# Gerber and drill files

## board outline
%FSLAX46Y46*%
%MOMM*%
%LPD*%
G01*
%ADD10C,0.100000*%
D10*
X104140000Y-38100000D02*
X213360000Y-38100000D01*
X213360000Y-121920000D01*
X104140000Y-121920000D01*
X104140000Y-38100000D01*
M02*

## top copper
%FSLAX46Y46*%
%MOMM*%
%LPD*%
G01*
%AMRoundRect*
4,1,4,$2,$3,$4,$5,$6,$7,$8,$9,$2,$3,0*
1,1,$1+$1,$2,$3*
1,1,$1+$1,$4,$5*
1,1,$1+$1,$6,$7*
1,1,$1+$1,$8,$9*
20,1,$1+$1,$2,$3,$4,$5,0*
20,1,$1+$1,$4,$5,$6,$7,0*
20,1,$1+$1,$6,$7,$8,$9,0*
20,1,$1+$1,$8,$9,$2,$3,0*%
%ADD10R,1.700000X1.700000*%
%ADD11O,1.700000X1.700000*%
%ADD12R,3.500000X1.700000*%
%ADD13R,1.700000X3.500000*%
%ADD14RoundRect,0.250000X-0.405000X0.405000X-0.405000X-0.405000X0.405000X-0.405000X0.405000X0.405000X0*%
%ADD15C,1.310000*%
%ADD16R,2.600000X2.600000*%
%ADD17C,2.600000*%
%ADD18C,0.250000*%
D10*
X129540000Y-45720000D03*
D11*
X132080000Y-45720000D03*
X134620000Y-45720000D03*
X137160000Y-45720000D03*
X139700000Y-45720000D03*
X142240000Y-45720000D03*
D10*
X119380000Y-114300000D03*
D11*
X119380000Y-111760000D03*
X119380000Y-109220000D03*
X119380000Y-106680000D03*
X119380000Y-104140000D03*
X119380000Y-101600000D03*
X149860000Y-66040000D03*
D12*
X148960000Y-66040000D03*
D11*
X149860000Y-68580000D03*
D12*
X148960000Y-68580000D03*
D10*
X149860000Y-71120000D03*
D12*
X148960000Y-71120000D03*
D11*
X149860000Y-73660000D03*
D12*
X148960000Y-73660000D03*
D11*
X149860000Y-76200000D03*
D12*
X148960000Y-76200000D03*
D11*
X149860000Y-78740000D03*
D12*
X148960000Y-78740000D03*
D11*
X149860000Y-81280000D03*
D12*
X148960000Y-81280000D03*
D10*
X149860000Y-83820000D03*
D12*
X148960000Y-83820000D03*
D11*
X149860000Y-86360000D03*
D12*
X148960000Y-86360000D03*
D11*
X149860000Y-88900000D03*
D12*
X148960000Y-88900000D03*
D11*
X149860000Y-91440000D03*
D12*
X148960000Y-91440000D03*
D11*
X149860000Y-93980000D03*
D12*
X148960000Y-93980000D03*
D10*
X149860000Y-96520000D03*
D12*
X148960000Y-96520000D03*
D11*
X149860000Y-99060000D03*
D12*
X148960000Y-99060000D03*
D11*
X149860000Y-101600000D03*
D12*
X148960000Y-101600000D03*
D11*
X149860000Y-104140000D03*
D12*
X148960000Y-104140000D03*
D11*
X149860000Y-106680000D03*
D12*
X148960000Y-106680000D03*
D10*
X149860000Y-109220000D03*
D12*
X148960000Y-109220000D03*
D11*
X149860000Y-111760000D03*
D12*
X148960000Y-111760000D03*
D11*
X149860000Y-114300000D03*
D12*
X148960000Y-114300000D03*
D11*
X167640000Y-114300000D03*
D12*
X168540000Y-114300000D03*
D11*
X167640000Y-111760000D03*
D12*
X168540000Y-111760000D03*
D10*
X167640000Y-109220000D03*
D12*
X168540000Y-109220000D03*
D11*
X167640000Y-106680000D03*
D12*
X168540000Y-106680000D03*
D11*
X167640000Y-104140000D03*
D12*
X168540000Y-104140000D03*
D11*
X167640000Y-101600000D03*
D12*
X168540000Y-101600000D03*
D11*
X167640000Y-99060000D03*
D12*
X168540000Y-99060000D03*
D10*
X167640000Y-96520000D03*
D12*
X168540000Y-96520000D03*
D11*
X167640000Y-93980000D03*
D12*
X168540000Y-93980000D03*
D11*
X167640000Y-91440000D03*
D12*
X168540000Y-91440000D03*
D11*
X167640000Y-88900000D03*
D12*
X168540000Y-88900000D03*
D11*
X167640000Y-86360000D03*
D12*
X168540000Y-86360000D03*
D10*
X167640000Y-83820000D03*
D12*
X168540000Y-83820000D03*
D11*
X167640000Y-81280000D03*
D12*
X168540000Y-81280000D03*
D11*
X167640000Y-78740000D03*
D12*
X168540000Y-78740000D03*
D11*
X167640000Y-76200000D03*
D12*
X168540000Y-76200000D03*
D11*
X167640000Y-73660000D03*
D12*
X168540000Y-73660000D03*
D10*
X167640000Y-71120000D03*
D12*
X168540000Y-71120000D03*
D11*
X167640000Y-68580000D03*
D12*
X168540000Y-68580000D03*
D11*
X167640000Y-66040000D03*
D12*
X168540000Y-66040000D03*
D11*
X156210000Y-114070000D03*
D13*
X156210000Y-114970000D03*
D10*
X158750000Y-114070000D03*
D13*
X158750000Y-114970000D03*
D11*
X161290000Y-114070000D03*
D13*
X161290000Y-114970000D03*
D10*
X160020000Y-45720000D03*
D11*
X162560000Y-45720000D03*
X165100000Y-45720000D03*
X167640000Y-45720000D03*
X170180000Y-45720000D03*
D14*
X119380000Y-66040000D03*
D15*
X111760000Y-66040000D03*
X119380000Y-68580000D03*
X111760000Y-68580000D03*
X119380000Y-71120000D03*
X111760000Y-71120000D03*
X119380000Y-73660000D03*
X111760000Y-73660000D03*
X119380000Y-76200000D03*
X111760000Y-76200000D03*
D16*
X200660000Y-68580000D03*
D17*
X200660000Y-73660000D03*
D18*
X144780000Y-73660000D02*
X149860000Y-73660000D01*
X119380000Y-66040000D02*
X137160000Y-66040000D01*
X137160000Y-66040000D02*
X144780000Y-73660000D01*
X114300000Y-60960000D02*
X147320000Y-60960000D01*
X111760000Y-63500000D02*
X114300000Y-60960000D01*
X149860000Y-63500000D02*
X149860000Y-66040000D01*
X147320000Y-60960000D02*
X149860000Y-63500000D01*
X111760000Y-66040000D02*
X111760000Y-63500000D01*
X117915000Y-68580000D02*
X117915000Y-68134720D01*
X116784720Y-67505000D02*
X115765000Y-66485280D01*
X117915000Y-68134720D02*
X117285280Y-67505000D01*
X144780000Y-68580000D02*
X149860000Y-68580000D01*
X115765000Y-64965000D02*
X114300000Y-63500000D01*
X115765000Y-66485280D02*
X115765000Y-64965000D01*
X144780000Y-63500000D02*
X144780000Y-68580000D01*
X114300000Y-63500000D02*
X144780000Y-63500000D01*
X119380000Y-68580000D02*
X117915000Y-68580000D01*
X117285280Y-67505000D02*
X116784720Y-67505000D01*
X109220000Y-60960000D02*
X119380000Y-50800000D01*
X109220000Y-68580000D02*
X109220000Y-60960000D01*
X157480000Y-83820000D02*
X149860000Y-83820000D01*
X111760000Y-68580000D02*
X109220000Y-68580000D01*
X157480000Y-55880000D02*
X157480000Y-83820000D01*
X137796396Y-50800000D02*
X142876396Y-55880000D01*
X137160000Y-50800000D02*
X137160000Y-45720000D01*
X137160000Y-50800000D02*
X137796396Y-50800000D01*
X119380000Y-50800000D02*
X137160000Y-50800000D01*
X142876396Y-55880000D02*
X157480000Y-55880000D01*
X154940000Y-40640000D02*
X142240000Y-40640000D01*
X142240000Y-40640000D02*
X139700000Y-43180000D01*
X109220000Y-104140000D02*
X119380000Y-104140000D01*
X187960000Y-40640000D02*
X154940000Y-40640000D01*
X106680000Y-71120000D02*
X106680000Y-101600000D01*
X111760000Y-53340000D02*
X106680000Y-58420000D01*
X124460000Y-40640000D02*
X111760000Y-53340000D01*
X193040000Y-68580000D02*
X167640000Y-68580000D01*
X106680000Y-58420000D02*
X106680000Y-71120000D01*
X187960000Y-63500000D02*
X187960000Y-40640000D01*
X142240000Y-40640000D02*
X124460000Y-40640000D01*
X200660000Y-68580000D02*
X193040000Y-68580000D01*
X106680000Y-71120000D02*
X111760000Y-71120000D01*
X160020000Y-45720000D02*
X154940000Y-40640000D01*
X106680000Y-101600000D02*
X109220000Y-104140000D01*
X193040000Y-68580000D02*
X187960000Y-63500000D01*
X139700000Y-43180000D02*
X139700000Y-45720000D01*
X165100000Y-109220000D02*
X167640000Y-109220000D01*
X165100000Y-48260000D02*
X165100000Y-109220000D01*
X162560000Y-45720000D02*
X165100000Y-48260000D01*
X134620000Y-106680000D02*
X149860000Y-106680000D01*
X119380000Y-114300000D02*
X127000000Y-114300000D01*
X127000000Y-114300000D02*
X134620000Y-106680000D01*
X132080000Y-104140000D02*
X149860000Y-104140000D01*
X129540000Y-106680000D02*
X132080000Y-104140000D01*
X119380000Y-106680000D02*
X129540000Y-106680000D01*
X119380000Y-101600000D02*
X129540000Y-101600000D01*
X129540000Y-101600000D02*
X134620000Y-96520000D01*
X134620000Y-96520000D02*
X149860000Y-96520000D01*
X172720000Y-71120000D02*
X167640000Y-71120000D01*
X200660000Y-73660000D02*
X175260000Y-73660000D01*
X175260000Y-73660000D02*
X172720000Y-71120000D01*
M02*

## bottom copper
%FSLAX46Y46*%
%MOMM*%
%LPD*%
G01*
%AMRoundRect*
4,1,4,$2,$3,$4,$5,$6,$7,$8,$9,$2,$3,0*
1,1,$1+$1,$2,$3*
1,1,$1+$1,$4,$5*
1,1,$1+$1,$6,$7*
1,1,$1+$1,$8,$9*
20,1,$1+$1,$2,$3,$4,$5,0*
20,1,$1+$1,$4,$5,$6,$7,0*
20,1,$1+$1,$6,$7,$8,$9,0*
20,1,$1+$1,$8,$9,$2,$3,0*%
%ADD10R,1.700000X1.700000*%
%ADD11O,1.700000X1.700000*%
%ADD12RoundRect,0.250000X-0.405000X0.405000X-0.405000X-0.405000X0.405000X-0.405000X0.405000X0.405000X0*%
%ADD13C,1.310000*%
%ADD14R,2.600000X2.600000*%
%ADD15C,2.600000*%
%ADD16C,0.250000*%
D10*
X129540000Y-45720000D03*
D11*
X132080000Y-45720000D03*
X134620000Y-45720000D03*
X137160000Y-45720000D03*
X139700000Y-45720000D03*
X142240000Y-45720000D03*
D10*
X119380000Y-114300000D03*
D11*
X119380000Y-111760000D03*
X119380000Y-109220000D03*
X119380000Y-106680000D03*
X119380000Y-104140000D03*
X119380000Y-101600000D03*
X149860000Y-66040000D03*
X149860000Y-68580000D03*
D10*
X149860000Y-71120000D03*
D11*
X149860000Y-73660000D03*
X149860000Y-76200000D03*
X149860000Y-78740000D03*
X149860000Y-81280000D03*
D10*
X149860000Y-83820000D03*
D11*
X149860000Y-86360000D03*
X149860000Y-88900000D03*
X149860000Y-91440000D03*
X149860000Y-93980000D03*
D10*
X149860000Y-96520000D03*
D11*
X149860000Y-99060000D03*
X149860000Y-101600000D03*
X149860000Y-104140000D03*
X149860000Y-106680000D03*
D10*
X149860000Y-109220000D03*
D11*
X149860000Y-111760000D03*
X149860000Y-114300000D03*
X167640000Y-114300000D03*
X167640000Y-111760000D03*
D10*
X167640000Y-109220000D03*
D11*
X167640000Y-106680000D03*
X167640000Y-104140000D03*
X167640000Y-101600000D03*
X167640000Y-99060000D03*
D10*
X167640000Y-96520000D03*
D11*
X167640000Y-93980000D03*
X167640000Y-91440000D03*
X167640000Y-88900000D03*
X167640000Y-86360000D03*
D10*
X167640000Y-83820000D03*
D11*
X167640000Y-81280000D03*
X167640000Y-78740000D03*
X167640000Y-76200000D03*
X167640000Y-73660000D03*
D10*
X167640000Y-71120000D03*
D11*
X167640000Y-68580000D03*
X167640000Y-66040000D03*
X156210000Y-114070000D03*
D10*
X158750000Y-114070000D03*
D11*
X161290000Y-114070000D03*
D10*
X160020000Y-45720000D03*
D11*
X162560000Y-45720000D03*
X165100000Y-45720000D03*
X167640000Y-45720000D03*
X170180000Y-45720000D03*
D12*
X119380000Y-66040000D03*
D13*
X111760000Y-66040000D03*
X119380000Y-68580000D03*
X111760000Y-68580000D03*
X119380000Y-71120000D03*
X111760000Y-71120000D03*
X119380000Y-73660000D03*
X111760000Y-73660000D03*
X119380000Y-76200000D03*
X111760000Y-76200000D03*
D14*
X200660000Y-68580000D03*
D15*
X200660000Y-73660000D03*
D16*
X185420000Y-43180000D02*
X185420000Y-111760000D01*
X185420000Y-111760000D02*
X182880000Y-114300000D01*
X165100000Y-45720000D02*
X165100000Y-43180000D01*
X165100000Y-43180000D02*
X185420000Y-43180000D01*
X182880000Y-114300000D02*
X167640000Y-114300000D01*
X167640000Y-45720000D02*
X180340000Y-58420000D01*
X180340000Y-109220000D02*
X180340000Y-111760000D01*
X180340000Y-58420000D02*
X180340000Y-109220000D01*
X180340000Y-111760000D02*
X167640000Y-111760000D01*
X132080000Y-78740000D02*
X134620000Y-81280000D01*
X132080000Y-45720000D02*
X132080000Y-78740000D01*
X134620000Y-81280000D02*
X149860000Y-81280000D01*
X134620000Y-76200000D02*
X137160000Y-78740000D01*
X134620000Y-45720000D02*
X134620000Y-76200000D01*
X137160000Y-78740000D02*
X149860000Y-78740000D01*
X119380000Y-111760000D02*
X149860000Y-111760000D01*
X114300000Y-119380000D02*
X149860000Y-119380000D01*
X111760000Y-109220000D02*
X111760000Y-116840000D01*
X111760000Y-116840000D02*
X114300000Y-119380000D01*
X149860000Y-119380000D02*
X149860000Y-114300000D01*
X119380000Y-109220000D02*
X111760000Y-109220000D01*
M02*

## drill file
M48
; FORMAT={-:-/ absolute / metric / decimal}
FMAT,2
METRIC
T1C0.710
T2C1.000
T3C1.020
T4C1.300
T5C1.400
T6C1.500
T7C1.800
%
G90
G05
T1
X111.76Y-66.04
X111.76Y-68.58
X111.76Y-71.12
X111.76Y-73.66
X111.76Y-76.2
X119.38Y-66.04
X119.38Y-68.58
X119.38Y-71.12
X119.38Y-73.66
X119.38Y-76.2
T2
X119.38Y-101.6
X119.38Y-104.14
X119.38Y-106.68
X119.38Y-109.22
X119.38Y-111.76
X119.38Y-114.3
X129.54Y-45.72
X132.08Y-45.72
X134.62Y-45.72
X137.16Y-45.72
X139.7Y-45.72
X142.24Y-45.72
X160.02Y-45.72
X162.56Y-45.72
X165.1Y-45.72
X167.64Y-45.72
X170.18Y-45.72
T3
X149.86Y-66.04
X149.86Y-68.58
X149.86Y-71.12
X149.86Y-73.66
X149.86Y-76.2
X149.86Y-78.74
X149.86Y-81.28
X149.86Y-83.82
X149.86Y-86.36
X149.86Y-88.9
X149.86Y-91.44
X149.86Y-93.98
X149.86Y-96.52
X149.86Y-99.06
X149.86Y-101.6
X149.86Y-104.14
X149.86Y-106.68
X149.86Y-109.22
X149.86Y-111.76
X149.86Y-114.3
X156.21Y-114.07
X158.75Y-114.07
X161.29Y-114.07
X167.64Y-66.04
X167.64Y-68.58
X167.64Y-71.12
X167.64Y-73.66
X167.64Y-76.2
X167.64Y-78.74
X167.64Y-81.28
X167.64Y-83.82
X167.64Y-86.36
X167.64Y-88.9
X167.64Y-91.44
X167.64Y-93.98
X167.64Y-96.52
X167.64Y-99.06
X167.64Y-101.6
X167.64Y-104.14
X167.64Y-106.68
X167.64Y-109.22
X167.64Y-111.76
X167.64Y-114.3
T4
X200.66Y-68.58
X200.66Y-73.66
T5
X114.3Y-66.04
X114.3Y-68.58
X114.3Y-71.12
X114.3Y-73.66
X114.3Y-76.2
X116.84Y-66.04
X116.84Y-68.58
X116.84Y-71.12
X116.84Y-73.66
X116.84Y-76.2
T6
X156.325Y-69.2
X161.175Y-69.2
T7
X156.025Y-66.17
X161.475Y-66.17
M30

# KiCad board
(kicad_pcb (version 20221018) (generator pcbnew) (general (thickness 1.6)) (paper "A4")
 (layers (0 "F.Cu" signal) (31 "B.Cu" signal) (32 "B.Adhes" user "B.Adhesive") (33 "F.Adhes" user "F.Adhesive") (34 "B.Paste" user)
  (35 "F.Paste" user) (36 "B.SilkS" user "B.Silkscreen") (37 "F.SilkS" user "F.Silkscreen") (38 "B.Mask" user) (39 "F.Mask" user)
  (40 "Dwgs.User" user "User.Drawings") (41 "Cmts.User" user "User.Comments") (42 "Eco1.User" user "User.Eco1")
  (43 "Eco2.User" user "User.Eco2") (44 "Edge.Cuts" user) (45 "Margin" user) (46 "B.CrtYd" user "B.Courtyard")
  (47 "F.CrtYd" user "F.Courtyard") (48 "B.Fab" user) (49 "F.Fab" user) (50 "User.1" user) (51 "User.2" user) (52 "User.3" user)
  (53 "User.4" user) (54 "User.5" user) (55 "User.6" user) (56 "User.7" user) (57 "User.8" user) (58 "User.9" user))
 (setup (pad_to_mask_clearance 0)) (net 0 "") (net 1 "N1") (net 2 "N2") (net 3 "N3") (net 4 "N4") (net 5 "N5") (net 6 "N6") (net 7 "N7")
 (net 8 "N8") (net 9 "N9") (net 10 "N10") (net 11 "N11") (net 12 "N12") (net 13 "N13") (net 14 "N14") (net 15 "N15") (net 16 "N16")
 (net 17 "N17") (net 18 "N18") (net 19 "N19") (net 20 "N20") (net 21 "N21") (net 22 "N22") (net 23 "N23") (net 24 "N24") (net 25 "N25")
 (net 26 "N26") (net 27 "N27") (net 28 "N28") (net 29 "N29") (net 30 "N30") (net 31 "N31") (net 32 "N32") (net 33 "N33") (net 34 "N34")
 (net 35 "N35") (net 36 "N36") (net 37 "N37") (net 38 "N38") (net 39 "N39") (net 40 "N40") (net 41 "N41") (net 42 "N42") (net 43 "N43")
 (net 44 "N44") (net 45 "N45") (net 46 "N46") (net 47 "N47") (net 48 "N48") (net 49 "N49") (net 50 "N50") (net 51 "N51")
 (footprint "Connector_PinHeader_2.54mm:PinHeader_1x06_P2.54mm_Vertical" (layer "F.Cu") (at 129.54 45.72 90)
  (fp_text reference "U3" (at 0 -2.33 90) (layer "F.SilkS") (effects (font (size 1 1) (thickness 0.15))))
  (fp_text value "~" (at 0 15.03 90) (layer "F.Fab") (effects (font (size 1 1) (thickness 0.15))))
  (pad "1" thru_hole rect (at 0 0 90) (size 1.7 1.7) (drill 1) (layers "*.Cu" "*.Mask") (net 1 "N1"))
  (pad "2" thru_hole oval (at 0 2.54 90) (size 1.7 1.7) (drill 1) (layers "*.Cu" "*.Mask") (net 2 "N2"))
  (pad "3" thru_hole oval (at 0 5.08 90) (size 1.7 1.7) (drill 1) (layers "*.Cu" "*.Mask") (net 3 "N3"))
  (pad "4" thru_hole oval (at 0 7.62 90) (size 1.7 1.7) (drill 1) (layers "*.Cu" "*.Mask") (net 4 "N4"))
  (pad "5" thru_hole oval (at 0 10.16 90) (size 1.7 1.7) (drill 1) (layers "*.Cu" "*.Mask") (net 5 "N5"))
  (pad "6" thru_hole oval (at 0 12.7 90) (size 1.7 1.7) (drill 1) (layers "*.Cu" "*.Mask") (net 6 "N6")))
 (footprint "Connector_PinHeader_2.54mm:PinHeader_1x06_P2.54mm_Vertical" (layer "F.Cu") (at 119.38 114.3 180)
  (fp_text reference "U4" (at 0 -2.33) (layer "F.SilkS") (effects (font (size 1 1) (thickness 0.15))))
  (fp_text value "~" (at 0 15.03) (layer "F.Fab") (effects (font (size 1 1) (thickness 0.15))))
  (pad "1" thru_hole rect (at 0 0 180) (size 1.7 1.7) (drill 1) (layers "*.Cu" "*.Mask") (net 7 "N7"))
  (pad "2" thru_hole oval (at 0 2.54 180) (size 1.7 1.7) (drill 1) (layers "*.Cu" "*.Mask") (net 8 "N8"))
  (pad "3" thru_hole oval (at 0 5.08 180) (size 1.7 1.7) (drill 1) (layers "*.Cu" "*.Mask") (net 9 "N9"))
  (pad "4" thru_hole oval (at 0 7.62 180) (size 1.7 1.7) (drill 1) (layers "*.Cu" "*.Mask") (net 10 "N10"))
  (pad "5" thru_hole oval (at 0 10.16 180) (size 1.7 1.7) (drill 1) (layers "*.Cu" "*.Mask") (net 5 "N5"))
  (pad "6" thru_hole oval (at 0 12.7 180) (size 1.7 1.7) (drill 1) (layers "*.Cu" "*.Mask") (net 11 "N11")))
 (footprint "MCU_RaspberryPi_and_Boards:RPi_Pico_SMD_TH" (layer "F.Cu") (at 158.75 90.17)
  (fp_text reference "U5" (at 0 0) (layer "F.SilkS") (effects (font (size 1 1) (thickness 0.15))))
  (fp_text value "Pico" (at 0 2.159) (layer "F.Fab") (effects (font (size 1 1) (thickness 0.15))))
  (pad "" np_thru_hole oval (at -2.725 -24) (size 1.8 1.8) (drill 1.8) (layers "*.Cu" "*.Mask"))
  (pad "" np_thru_hole oval (at -2.425 -20.97) (size 1.5 1.5) (drill 1.5) (layers "*.Cu" "*.Mask"))
  (pad "" np_thru_hole oval (at 2.425 -20.97) (size 1.5 1.5) (drill 1.5) (layers "*.Cu" "*.Mask"))
  (pad "" np_thru_hole oval (at 2.725 -24) (size 1.8 1.8) (drill 1.8) (layers "*.Cu" "*.Mask"))
  (pad "1" thru_hole oval (at -8.89 -24.13) (size 1.7 1.7) (drill 1.02) (layers "*.Cu" "*.Mask") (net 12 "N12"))
  (pad "1" smd rect (at -8.89 -24.13) (size 3.5 1.7) (drill (offset -0.9 0)) (layers "F.Cu" "F.Mask") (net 12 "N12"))
  (pad "2" thru_hole oval (at -8.89 -21.59) (size 1.7 1.7) (drill 1.02) (layers "*.Cu" "*.Mask") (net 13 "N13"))
  (pad "2" smd rect (at -8.89 -21.59) (size 3.5 1.7) (drill (offset -0.9 0)) (layers "F.Cu" "F.Mask") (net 13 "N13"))
  (pad "3" thru_hole rect (at -8.89 -19.05) (size 1.7 1.7) (drill 1.02) (layers "*.Cu" "*.Mask") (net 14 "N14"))
  (pad "3" smd rect (at -8.89 -19.05) (size 3.5 1.7) (drill (offset -0.9 0)) (layers "F.Cu" "F.Mask") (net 14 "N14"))
  (pad "4" thru_hole oval (at -8.89 -16.51) (size 1.7 1.7) (drill 1.02) (layers "*.Cu" "*.Mask") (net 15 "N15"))
  (pad "4" smd rect (at -8.89 -16.51) (size 3.5 1.7) (drill (offset -0.9 0)) (layers "F.Cu" "F.Mask") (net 15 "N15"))
  (pad "5" thru_hole oval (at -8.89 -13.97) (size 1.7 1.7) (drill 1.02) (layers "*.Cu" "*.Mask") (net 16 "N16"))
  (pad "5" smd rect (at -8.89 -13.97) (size 3.5 1.7) (drill (offset -0.9 0)) (layers "F.Cu" "F.Mask") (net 16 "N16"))
  (pad "6" thru_hole oval (at -8.89 -11.43) (size 1.7 1.7) (drill 1.02) (layers "*.Cu" "*.Mask") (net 3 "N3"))
  (pad "6" smd rect (at -8.89 -11.43) (size 3.5 1.7) (drill (offset -0.9 0)) (layers "F.Cu" "F.Mask") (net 3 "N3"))
  (pad "7" thru_hole oval (at -8.89 -8.89) (size 1.7 1.7) (drill 1.02) (layers "*.Cu" "*.Mask") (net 2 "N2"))
  (pad "7" smd rect (at -8.89 -8.89) (size 3.5 1.7) (drill (offset -0.9 0)) (layers "F.Cu" "F.Mask") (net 2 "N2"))
  (pad "8" thru_hole rect (at -8.89 -6.35) (size 1.7 1.7) (drill 1.02) (layers "*.Cu" "*.Mask") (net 4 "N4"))
  (pad "8" smd rect (at -8.89 -6.35) (size 3.5 1.7) (drill (offset -0.9 0)) (layers "F.Cu" "F.Mask") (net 4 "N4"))
  (pad "9" thru_hole oval (at -8.89 -3.81) (size 1.7 1.7) (drill 1.02) (layers "*.Cu" "*.Mask") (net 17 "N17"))
  (pad "9" smd rect (at -8.89 -3.81) (size 3.5 1.7) (drill (offset -0.9 0)) (layers "F.Cu" "F.Mask") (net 17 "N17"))
  (pad "10" thru_hole oval (at -8.89 -1.27) (size 1.7 1.7) (drill 1.02) (layers "*.Cu" "*.Mask") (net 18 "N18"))
  (pad "10" smd rect (at -8.89 -1.27) (size 3.5 1.7) (drill (offset -0.9 0)) (layers "F.Cu" "F.Mask") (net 18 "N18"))
  (pad "11" thru_hole oval (at -8.89 1.27) (size 1.7 1.7) (drill 1.02) (layers "*.Cu" "*.Mask") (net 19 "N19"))
  (pad "11" smd rect (at -8.89 1.27) (size 3.5 1.7) (drill (offset -0.9 0)) (layers "F.Cu" "F.Mask") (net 19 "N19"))
  (pad "12" thru_hole oval (at -8.89 3.81) (size 1.7 1.7) (drill 1.02) (layers "*.Cu" "*.Mask") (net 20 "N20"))
  (pad "12" smd rect (at -8.89 3.81) (size 3.5 1.7) (drill (offset -0.9 0)) (layers "F.Cu" "F.Mask") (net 20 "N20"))
  (pad "13" thru_hole rect (at -8.89 6.35) (size 1.7 1.7) (drill 1.02) (layers "*.Cu" "*.Mask") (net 11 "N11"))
  (pad "13" smd rect (at -8.89 6.35) (size 3.5 1.7) (drill (offset -0.9 0)) (layers "F.Cu" "F.Mask") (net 11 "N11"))
  (pad "14" thru_hole oval (at -8.89 8.89) (size 1.7 1.7) (drill 1.02) (layers "*.Cu" "*.Mask") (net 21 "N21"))
  (pad "14" smd rect (at -8.89 8.89) (size 3.5 1.7) (drill (offset -0.9 0)) (layers "F.Cu" "F.Mask") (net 21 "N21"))
  (pad "15" thru_hole oval (at -8.89 11.43) (size 1.7 1.7) (drill 1.02) (layers "*.Cu" "*.Mask") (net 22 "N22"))
  (pad "15" smd rect (at -8.89 11.43) (size 3.5 1.7) (drill (offset -0.9 0)) (layers "F.Cu" "F.Mask") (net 22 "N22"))
  (pad "16" thru_hole oval (at -8.89 13.97) (size 1.7 1.7) (drill 1.02) (layers "*.Cu" "*.Mask") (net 10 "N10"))
  (pad "16" smd rect (at -8.89 13.97) (size 3.5 1.7) (drill (offset -0.9 0)) (layers "F.Cu" "F.Mask") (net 10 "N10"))
  (pad "17" thru_hole oval (at -8.89 16.51) (size 1.7 1.7) (drill 1.02) (layers "*.Cu" "*.Mask") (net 7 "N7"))
  (pad "17" smd rect (at -8.89 16.51) (size 3.5 1.7) (drill (offset -0.9 0)) (layers "F.Cu" "F.Mask") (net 7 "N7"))
  (pad "18" thru_hole rect (at -8.89 19.05) (size 1.7 1.7) (drill 1.02) (layers "*.Cu" "*.Mask") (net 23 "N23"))
  (pad "18" smd rect (at -8.89 19.05) (size 3.5 1.7) (drill (offset -0.9 0)) (layers "F.Cu" "F.Mask") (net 23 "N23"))
  (pad "19" thru_hole oval (at -8.89 21.59) (size 1.7 1.7) (drill 1.02) (layers "*.Cu" "*.Mask") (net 8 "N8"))
  (pad "19" smd rect (at -8.89 21.59) (size 3.5 1.7) (drill (offset -0.9 0)) (layers "F.Cu" "F.Mask") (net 8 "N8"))
  (pad "20" thru_hole oval (at -8.89 24.13) (size 1.7 1.7) (drill 1.02) (layers "*.Cu" "*.Mask") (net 9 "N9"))
  (pad "20" smd rect (at -8.89 24.13) (size 3.5 1.7) (drill (offset -0.9 0)) (layers "F.Cu" "F.Mask") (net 9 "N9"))
  (pad "21" thru_hole oval (at 8.89 24.13) (size 1.7 1.7) (drill 1.02) (layers "*.Cu" "*.Mask") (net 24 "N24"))
  (pad "21" smd rect (at 8.89 24.13) (size 3.5 1.7) (drill (offset 0.9 0)) (layers "F.Cu" "F.Mask") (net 24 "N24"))
  (pad "22" thru_hole oval (at 8.89 21.59) (size 1.7 1.7) (drill 1.02) (layers "*.Cu" "*.Mask") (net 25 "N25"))
  (pad "22" smd rect (at 8.89 21.59) (size 3.5 1.7) (drill (offset 0.9 0)) (layers "F.Cu" "F.Mask") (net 25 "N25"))
  (pad "23" thru_hole rect (at 8.89 19.05) (size 1.7 1.7) (drill 1.02) (layers "*.Cu" "*.Mask") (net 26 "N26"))
  (pad "23" smd rect (at 8.89 19.05) (size 3.5 1.7) (drill (offset 0.9 0)) (layers "F.Cu" "F.Mask") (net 26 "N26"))
  (pad "24" thru_hole oval (at 8.89 16.51) (size 1.7 1.7) (drill 1.02) (layers "*.Cu" "*.Mask") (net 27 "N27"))
  (pad "24" smd rect (at 8.89 16.51) (size 3.5 1.7) (drill (offset 0.9 0)) (layers "F.Cu" "F.Mask") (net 27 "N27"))
  (pad "25" thru_hole oval (at 8.89 13.97) (size 1.7 1.7) (drill 1.02) (layers "*.Cu" "*.Mask") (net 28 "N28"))
  (pad "25" smd rect (at 8.89 13.97) (size 3.5 1.7) (drill (offset 0.9 0)) (layers "F.Cu" "F.Mask") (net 28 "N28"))
  (pad "26" thru_hole oval (at 8.89 11.43) (size 1.7 1.7) (drill 1.02) (layers "*.Cu" "*.Mask") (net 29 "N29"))
  (pad "26" smd rect (at 8.89 11.43) (size 3.5 1.7) (drill (offset 0.9 0)) (layers "F.Cu" "F.Mask") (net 29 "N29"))
  (pad "27" thru_hole oval (at 8.89 8.89) (size 1.7 1.7) (drill 1.02) (layers "*.Cu" "*.Mask") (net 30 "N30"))
  (pad "27" smd rect (at 8.89 8.89) (size 3.5 1.7) (drill (offset 0.9 0)) (layers "F.Cu" "F.Mask") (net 30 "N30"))
  (pad "28" thru_hole rect (at 8.89 6.35) (size 1.7 1.7) (drill 1.02) (layers "*.Cu" "*.Mask") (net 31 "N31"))
  (pad "28" smd rect (at 8.89 6.35) (size 3.5 1.7) (drill (offset 0.9 0)) (layers "F.Cu" "F.Mask") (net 31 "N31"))
  (pad "29" thru_hole oval (at 8.89 3.81) (size 1.7 1.7) (drill 1.02) (layers "*.Cu" "*.Mask") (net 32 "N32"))
  (pad "29" smd rect (at 8.89 3.81) (size 3.5 1.7) (drill (offset 0.9 0)) (layers "F.Cu" "F.Mask") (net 32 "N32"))
  (pad "30" thru_hole oval (at 8.89 1.27) (size 1.7 1.7) (drill 1.02) (layers "*.Cu" "*.Mask") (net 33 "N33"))
  (pad "30" smd rect (at 8.89 1.27) (size 3.5 1.7) (drill (offset 0.9 0)) (layers "F.Cu" "F.Mask") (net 33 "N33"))
  (pad "31" thru_hole oval (at 8.89 -1.27) (size 1.7 1.7) (drill 1.02) (layers "*.Cu" "*.Mask") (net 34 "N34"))
  (pad "31" smd rect (at 8.89 -1.27) (size 3.5 1.7) (drill (offset 0.9 0)) (layers "F.Cu" "F.Mask") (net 34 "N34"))
  (pad "32" thru_hole oval (at 8.89 -3.81) (size 1.7 1.7) (drill 1.02) (layers "*.Cu" "*.Mask") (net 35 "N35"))
  (pad "32" smd rect (at 8.89 -3.81) (size 3.5 1.7) (drill (offset 0.9 0)) (layers "F.Cu" "F.Mask") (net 35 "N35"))
  (pad "33" thru_hole rect (at 8.89 -6.35) (size 1.7 1.7) (drill 1.02) (layers "*.Cu" "*.Mask") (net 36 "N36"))
  (pad "33" smd rect (at 8.89 -6.35) (size 3.5 1.7) (drill (offset 0.9 0)) (layers "F.Cu" "F.Mask") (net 36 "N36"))
  (pad "34" thru_hole oval (at 8.89 -8.89) (size 1.7 1.7) (drill 1.02) (layers "*.Cu" "*.Mask") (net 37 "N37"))
  (pad "34" smd rect (at 8.89 -8.89) (size 3.5 1.7) (drill (offset 0.9 0)) (layers "F.Cu" "F.Mask") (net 37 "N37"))
  (pad "35" thru_hole oval (at 8.89 -11.43) (size 1.7 1.7) (drill 1.02) (layers "*.Cu" "*.Mask") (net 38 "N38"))
  (pad "35" smd rect (at 8.89 -11.43) (size 3.5 1.7) (drill (offset 0.9 0)) (layers "F.Cu" "F.Mask") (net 38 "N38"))
  (pad "36" thru_hole oval (at 8.89 -13.97) (size 1.7 1.7) (drill 1.02) (layers "*.Cu" "*.Mask") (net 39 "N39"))
  (pad "36" smd rect (at 8.89 -13.97) (size 3.5 1.7) (drill (offset 0.9 0)) (layers "F.Cu" "F.Mask") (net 39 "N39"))
  (pad "37" thru_hole oval (at 8.89 -16.51) (size 1.7 1.7) (drill 1.02) (layers "*.Cu" "*.Mask") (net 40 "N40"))
  (pad "37" smd rect (at 8.89 -16.51) (size 3.5 1.7) (drill (offset 0.9 0)) (layers "F.Cu" "F.Mask") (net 40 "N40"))
  (pad "38" thru_hole rect (at 8.89 -19.05) (size 1.7 1.7) (drill 1.02) (layers "*.Cu" "*.Mask") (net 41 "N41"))
  (pad "38" smd rect (at 8.89 -19.05) (size 3.5 1.7) (drill (offset 0.9 0)) (layers "F.Cu" "F.Mask") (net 41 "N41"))
  (pad "39" thru_hole oval (at 8.89 -21.59) (size 1.7 1.7) (drill 1.02) (layers "*.Cu" "*.Mask") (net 5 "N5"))
  (pad "39" smd rect (at 8.89 -21.59) (size 3.5 1.7) (drill (offset 0.9 0)) (layers "F.Cu" "F.Mask") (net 5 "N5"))
  (pad "40" thru_hole oval (at 8.89 -24.13) (size 1.7 1.7) (drill 1.02) (layers "*.Cu" "*.Mask") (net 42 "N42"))
  (pad "40" smd rect (at 8.89 -24.13) (size 3.5 1.7) (drill (offset 0.9 0)) (layers "F.Cu" "F.Mask") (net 42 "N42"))
  (pad "41" thru_hole oval (at -2.54 23.9) (size 1.7 1.7) (drill 1.02) (layers "*.Cu" "*.Mask") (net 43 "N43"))
  (pad "41" smd rect (at -2.54 23.9 90) (size 3.5 1.7) (drill (offset -0.9 0)) (layers "F.Cu" "F.Mask") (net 43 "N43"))
  (pad "42" thru_hole rect (at 0 23.9) (size 1.7 1.7) (drill 1.02) (layers "*.Cu" "*.Mask") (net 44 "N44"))
  (pad "42" smd rect (at 0 23.9 90) (size 3.5 1.7) (drill (offset -0.9 0)) (layers "F.Cu" "F.Mask") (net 44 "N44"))
  (pad "43" thru_hole oval (at 2.54 23.9) (size 1.7 1.7) (drill 1.02) (layers "*.Cu" "*.Mask") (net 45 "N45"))
  (pad "43" smd rect (at 2.54 23.9 90) (size 3.5 1.7) (drill (offset -0.9 0)) (layers "F.Cu" "F.Mask") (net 45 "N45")))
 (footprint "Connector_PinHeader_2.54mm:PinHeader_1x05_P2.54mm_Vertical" (layer "F.Cu") (at 160.02 45.72 90)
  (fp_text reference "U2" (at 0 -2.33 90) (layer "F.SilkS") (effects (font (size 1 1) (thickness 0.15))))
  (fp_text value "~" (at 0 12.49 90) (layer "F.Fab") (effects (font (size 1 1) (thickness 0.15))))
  (pad "1" thru_hole rect (at 0 0 90) (size 1.7 1.7) (drill 1) (layers "*.Cu" "*.Mask") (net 5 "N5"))
  (pad "2" thru_hole oval (at 0 2.54 90) (size 1.7 1.7) (drill 1) (layers "*.Cu" "*.Mask") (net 26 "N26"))
  (pad "3" thru_hole oval (at 0 5.08 90) (size 1.7 1.7) (drill 1) (layers "*.Cu" "*.Mask") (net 24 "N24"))
  (pad "4" thru_hole oval (at 0 7.62 90) (size 1.7 1.7) (drill 1) (layers "*.Cu" "*.Mask") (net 25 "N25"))
  (pad "5" thru_hole oval (at 0 10.16 90) (size 1.7 1.7) (drill 1) (layers "*.Cu" "*.Mask") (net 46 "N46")))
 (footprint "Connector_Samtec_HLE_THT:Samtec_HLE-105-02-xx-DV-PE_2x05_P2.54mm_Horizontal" (layer "F.Cu") (at 119.38 66.04 -90)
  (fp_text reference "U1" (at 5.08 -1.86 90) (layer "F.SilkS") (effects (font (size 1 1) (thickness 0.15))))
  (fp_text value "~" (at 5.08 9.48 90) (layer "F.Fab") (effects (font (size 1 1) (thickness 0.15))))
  (pad "" np_thru_hole circle (at 0 2.54 270) (size 1.4 1.4) (drill 1.4) (layers "*.Cu" "*.Mask"))
  (pad "" np_thru_hole circle (at 0 5.08 270) (size 1.4 1.4) (drill 1.4) (layers "*.Cu" "*.Mask"))
  (pad "" np_thru_hole circle (at 2.54 2.54 270) (size 1.4 1.4) (drill 1.4) (layers "*.Cu" "*.Mask"))
  (pad "" np_thru_hole circle (at 2.54 5.08 270) (size 1.4 1.4) (drill 1.4) (layers "*.Cu" "*.Mask"))
  (pad "" np_thru_hole circle (at 5.08 2.54 270) (size 1.4 1.4) (drill 1.4) (layers "*.Cu" "*.Mask"))
  (pad "" np_thru_hole circle (at 5.08 5.08 270) (size 1.4 1.4) (drill 1.4) (layers "*.Cu" "*.Mask"))
  (pad "" np_thru_hole circle (at 7.62 2.54 270) (size 1.4 1.4) (drill 1.4) (layers "*.Cu" "*.Mask"))
  (pad "" np_thru_hole circle (at 7.62 5.08 270) (size 1.4 1.4) (drill 1.4) (layers "*.Cu" "*.Mask"))
  (pad "" np_thru_hole circle (at 10.16 2.54 270) (size 1.4 1.4) (drill 1.4) (layers "*.Cu" "*.Mask"))
  (pad "" np_thru_hole circle (at 10.16 5.08 270) (size 1.4 1.4) (drill 1.4) (layers "*.Cu" "*.Mask"))
  (pad "1" thru_hole roundrect (at 0 0 270) (size 1.31 1.31) (drill 0.71) (layers "*.Cu" "*.Mask") (roundrect_rratio 0.1908396947)
   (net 15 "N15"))
  (pad "2" thru_hole circle (at 0 7.62 270) (size 1.31 1.31) (drill 0.71) (layers "*.Cu" "*.Mask") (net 12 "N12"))
  (pad "3" thru_hole circle (at 2.54 0 270) (size 1.31 1.31) (drill 0.71) (layers "*.Cu" "*.Mask") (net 13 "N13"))
  (pad "4" thru_hole circle (at 2.54 7.62 270) (size 1.31 1.31) (drill 0.71) (layers "*.Cu" "*.Mask") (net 4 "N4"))
  (pad "5" thru_hole circle (at 5.08 0 270) (size 1.31 1.31) (drill 0.71) (layers "*.Cu" "*.Mask") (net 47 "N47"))
  (pad "6" thru_hole circle (at 5.08 7.62 270) (size 1.31 1.31) (drill 0.71) (layers "*.Cu" "*.Mask") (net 5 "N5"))
  (pad "7" thru_hole circle (at 7.62 0 270) (size 1.31 1.31) (drill 0.71) (layers "*.Cu" "*.Mask") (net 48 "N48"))
  (pad "8" thru_hole circle (at 7.62 7.62 270) (size 1.31 1.31) (drill 0.71) (layers "*.Cu" "*.Mask") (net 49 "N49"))
  (pad "9" thru_hole circle (at 10.16 0 270) (size 1.31 1.31) (drill 0.71) (layers "*.Cu" "*.Mask") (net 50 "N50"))
  (pad "10" thru_hole circle (at 10.16 7.62 270) (size 1.31 1.31) (drill 0.71) (layers "*.Cu" "*.Mask") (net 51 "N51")))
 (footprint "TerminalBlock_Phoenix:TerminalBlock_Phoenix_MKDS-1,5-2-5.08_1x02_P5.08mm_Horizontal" (layer "F.Cu") (at 200.66 68.58 -90)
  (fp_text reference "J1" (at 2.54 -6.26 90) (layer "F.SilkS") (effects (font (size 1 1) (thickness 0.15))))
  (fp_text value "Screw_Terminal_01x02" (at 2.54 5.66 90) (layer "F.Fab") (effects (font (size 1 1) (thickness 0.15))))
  (pad "1" thru_hole rect (at 0 0 270) (size 2.6 2.6) (drill 1.3) (layers "*.Cu" "*.Mask") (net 5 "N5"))
  (pad "2" thru_hole circle (at 5.08 0 270) (size 2.6 2.6) (drill 1.3) (layers "*.Cu" "*.Mask") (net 41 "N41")))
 (gr_rect (start 104.14 38.1) (end 213.36 121.92) (stroke (width 0.1) (type default)) (fill none) (layer "Edge.Cuts"))
 (segment (start 144.78 73.66) (end 149.86 73.66) (width 0.25) (layer "F.Cu") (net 15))
 (segment (start 119.38 66.04) (end 137.16 66.04) (width 0.25) (layer "F.Cu") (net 15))
 (segment (start 137.16 66.04) (end 144.78 73.66) (width 0.25) (layer "F.Cu") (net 15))
 (segment (start 114.3 60.96) (end 147.32 60.96) (width 0.25) (layer "F.Cu") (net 12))
 (segment (start 111.76 63.5) (end 114.3 60.96) (width 0.25) (layer "F.Cu") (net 12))
 (segment (start 149.86 63.5) (end 149.86 66.04) (width 0.25) (layer "F.Cu") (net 12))
 (segment (start 147.32 60.96) (end 149.86 63.5) (width 0.25) (layer "F.Cu") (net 12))
 (segment (start 111.76 66.04) (end 111.76 63.5) (width 0.25) (layer "F.Cu") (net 12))
 (segment (start 117.915 68.58) (end 117.915 68.13472) (width 0.25) (layer "F.Cu") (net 13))
 (segment (start 116.78472 67.505) (end 115.765 66.48528) (width 0.25) (layer "F.Cu") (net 13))
 (segment (start 117.915 68.13472) (end 117.28528 67.505) (width 0.25) (layer "F.Cu") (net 13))
 (segment (start 144.78 68.58) (end 149.86 68.58) (width 0.25) (layer "F.Cu") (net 13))
 (segment (start 115.765 64.965) (end 114.3 63.5) (width 0.25) (layer "F.Cu") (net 13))
 (segment (start 115.765 66.48528) (end 115.765 64.965) (width 0.25) (layer "F.Cu") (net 13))
 (segment (start 144.78 63.5) (end 144.78 68.58) (width 0.25) (layer "F.Cu") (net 13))
 (segment (start 114.3 63.5) (end 144.78 63.5) (width 0.25) (layer "F.Cu") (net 13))
 (segment (start 119.38 68.58) (end 117.915 68.58) (width 0.25) (layer "F.Cu") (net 13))
 (segment (start 117.28528 67.505) (end 116.78472 67.505) (width 0.25) (layer "F.Cu") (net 13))
 (segment (start 109.22 60.96) (end 119.38 50.8) (width 0.25) (layer "F.Cu") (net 4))
 (segment (start 109.22 68.58) (end 109.22 60.96) (width 0.25) (layer "F.Cu") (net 4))
 (segment (start 157.48 83.82) (end 149.86 83.82) (width 0.25) (layer "F.Cu") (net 4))
 (segment (start 111.76 68.58) (end 109.22 68.58) (width 0.25) (layer "F.Cu") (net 4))
 (segment (start 157.48 55.88) (end 157.48 83.82) (width 0.25) (layer "F.Cu") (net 4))
 (segment (start 137.796396 50.8) (end 142.876396 55.88) (width 0.25) (layer "F.Cu") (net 4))
 (segment (start 137.16 50.8) (end 137.16 45.72) (width 0.25) (layer "F.Cu") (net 4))
 (segment (start 137.16 50.8) (end 137.796396 50.8) (width 0.25) (layer "F.Cu") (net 4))
 (segment (start 119.38 50.8) (end 137.16 50.8) (width 0.25) (layer "F.Cu") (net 4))
 (segment (start 142.876396 55.88) (end 157.48 55.88) (width 0.25) (layer "F.Cu") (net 4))
 (segment (start 154.94 40.64) (end 142.24 40.64) (width 0.25) (layer "F.Cu") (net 5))
 (segment (start 142.24 40.64) (end 139.7 43.18) (width 0.25) (layer "F.Cu") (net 5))
 (segment (start 109.22 104.14) (end 119.38 104.14) (width 0.25) (layer "F.Cu") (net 5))
 (segment (start 187.96 40.64) (end 154.94 40.64) (width 0.25) (layer "F.Cu") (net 5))
 (segment (start 106.68 71.12) (end 106.68 101.6) (width 0.25) (layer "F.Cu") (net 5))
 (segment (start 111.76 53.34) (end 106.68 58.42) (width 0.25) (layer "F.Cu") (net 5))
 (segment (start 124.46 40.64) (end 111.76 53.34) (width 0.25) (layer "F.Cu") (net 5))
 (segment (start 193.04 68.58) (end 167.64 68.58) (width 0.25) (layer "F.Cu") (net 5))
 (segment (start 106.68 58.42) (end 106.68 71.12) (width 0.25) (layer "F.Cu") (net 5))
 (segment (start 187.96 63.5) (end 187.96 40.64) (width 0.25) (layer "F.Cu") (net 5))
 (segment (start 142.24 40.64) (end 124.46 40.64) (width 0.25) (layer "F.Cu") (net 5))
 (segment (start 200.66 68.58) (end 193.04 68.58) (width 0.25) (layer "F.Cu") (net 5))
 (segment (start 106.68 71.12) (end 111.76 71.12) (width 0.25) (layer "F.Cu") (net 5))
 (segment (start 160.02 45.72) (end 154.94 40.64) (width 0.25) (layer "F.Cu") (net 5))
 (segment (start 106.68 101.6) (end 109.22 104.14) (width 0.25) (layer "F.Cu") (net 5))
 (segment (start 193.04 68.58) (end 187.96 63.5) (width 0.25) (layer "F.Cu") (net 5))
 (segment (start 139.7 43.18) (end 139.7 45.72) (width 0.25) (layer "F.Cu") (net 5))
 (segment (start 165.1 109.22) (end 167.64 109.22) (width 0.25) (layer "F.Cu") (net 26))
 (segment (start 165.1 48.26) (end 165.1 109.22) (width 0.25) (layer "F.Cu") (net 26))
 (segment (start 162.56 45.72) (end 165.1 48.26) (width 0.25) (layer "F.Cu") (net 26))
 (segment (start 185.42 43.18) (end 185.42 111.76) (width 0.25) (layer "B.Cu") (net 24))
 (segment (start 185.42 111.76) (end 182.88 114.3) (width 0.25) (layer "B.Cu") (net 24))
 (segment (start 165.1 45.72) (end 165.1 43.18) (width 0.25) (layer "B.Cu") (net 24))
 (segment (start 165.1 43.18) (end 185.42 43.18) (width 0.25) (layer "B.Cu") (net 24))
 (segment (start 182.88 114.3) (end 167.64 114.3) (width 0.25) (layer "B.Cu") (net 24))
 (segment (start 167.64 45.72) (end 180.34 58.42) (width 0.25) (layer "B.Cu") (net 25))
 (segment (start 180.34 109.22) (end 180.34 111.76) (width 0.25) (layer "B.Cu") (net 25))
 (segment (start 180.34 58.42) (end 180.34 109.22) (width 0.25) (layer "B.Cu") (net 25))
 (segment (start 180.34 111.76) (end 167.64 111.76) (width 0.25) (layer "B.Cu") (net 25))
 (segment (start 132.08 78.74) (end 134.62 81.28) (width 0.25) (layer "B.Cu") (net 2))
 (segment (start 132.08 45.72) (end 132.08 78.74) (width 0.25) (layer "B.Cu") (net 2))
 (segment (start 134.62 81.28) (end 149.86 81.28) (width 0.25) (layer "B.Cu") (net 2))
 (segment (start 134.62 76.2) (end 137.16 78.74) (width 0.25) (layer "B.Cu") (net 3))
 (segment (start 134.62 45.72) (end 134.62 76.2) (width 0.25) (layer "B.Cu") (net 3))
 (segment (start 137.16 78.74) (end 149.86 78.74) (width 0.25) (layer "B.Cu") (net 3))
 (segment (start 134.62 106.68) (end 149.86 106.68) (width 0.25) (layer "F.Cu") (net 7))
 (segment (start 119.38 114.3) (end 127 114.3) (width 0.25) (layer "F.Cu") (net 7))
 (segment (start 127 114.3) (end 134.62 106.68) (width 0.25) (layer "F.Cu") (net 7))
 (segment (start 119.38 111.76) (end 149.86 111.76) (width 0.25) (layer "B.Cu") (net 8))
 (segment (start 114.3 119.38) (end 149.86 119.38) (width 0.25) (layer "B.Cu") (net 9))
 (segment (start 111.76 109.22) (end 111.76 116.84) (width 0.25) (layer "B.Cu") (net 9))
 (segment (start 111.76 116.84) (end 114.3 119.38) (width 0.25) (layer "B.Cu") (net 9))
 (segment (start 149.86 119.38) (end 149.86 114.3) (width 0.25) (layer "B.Cu") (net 9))
 (segment (start 119.38 109.22) (end 111.76 109.22) (width 0.25) (layer "B.Cu") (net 9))
 (segment (start 132.08 104.14) (end 149.86 104.14) (width 0.25) (layer "F.Cu") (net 10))
 (segment (start 129.54 106.68) (end 132.08 104.14) (width 0.25) (layer "F.Cu") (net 10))
 (segment (start 119.38 106.68) (end 129.54 106.68) (width 0.25) (layer "F.Cu") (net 10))
 (segment (start 119.38 101.6) (end 129.54 101.6) (width 0.25) (layer "F.Cu") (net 11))
 (segment (start 129.54 101.6) (end 134.62 96.52) (width 0.25) (layer "F.Cu") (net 11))
 (segment (start 134.62 96.52) (end 149.86 96.52) (width 0.25) (layer "F.Cu") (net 11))
 (segment (start 172.72 71.12) (end 167.64 71.12) (width 0.25) (layer "F.Cu") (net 41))
 (segment (start 200.66 73.66) (end 175.26 73.66) (width 0.25) (layer "F.Cu") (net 41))
 (segment (start 175.26 73.66) (end 172.72 71.12) (width 0.25) (layer "F.Cu") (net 41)))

